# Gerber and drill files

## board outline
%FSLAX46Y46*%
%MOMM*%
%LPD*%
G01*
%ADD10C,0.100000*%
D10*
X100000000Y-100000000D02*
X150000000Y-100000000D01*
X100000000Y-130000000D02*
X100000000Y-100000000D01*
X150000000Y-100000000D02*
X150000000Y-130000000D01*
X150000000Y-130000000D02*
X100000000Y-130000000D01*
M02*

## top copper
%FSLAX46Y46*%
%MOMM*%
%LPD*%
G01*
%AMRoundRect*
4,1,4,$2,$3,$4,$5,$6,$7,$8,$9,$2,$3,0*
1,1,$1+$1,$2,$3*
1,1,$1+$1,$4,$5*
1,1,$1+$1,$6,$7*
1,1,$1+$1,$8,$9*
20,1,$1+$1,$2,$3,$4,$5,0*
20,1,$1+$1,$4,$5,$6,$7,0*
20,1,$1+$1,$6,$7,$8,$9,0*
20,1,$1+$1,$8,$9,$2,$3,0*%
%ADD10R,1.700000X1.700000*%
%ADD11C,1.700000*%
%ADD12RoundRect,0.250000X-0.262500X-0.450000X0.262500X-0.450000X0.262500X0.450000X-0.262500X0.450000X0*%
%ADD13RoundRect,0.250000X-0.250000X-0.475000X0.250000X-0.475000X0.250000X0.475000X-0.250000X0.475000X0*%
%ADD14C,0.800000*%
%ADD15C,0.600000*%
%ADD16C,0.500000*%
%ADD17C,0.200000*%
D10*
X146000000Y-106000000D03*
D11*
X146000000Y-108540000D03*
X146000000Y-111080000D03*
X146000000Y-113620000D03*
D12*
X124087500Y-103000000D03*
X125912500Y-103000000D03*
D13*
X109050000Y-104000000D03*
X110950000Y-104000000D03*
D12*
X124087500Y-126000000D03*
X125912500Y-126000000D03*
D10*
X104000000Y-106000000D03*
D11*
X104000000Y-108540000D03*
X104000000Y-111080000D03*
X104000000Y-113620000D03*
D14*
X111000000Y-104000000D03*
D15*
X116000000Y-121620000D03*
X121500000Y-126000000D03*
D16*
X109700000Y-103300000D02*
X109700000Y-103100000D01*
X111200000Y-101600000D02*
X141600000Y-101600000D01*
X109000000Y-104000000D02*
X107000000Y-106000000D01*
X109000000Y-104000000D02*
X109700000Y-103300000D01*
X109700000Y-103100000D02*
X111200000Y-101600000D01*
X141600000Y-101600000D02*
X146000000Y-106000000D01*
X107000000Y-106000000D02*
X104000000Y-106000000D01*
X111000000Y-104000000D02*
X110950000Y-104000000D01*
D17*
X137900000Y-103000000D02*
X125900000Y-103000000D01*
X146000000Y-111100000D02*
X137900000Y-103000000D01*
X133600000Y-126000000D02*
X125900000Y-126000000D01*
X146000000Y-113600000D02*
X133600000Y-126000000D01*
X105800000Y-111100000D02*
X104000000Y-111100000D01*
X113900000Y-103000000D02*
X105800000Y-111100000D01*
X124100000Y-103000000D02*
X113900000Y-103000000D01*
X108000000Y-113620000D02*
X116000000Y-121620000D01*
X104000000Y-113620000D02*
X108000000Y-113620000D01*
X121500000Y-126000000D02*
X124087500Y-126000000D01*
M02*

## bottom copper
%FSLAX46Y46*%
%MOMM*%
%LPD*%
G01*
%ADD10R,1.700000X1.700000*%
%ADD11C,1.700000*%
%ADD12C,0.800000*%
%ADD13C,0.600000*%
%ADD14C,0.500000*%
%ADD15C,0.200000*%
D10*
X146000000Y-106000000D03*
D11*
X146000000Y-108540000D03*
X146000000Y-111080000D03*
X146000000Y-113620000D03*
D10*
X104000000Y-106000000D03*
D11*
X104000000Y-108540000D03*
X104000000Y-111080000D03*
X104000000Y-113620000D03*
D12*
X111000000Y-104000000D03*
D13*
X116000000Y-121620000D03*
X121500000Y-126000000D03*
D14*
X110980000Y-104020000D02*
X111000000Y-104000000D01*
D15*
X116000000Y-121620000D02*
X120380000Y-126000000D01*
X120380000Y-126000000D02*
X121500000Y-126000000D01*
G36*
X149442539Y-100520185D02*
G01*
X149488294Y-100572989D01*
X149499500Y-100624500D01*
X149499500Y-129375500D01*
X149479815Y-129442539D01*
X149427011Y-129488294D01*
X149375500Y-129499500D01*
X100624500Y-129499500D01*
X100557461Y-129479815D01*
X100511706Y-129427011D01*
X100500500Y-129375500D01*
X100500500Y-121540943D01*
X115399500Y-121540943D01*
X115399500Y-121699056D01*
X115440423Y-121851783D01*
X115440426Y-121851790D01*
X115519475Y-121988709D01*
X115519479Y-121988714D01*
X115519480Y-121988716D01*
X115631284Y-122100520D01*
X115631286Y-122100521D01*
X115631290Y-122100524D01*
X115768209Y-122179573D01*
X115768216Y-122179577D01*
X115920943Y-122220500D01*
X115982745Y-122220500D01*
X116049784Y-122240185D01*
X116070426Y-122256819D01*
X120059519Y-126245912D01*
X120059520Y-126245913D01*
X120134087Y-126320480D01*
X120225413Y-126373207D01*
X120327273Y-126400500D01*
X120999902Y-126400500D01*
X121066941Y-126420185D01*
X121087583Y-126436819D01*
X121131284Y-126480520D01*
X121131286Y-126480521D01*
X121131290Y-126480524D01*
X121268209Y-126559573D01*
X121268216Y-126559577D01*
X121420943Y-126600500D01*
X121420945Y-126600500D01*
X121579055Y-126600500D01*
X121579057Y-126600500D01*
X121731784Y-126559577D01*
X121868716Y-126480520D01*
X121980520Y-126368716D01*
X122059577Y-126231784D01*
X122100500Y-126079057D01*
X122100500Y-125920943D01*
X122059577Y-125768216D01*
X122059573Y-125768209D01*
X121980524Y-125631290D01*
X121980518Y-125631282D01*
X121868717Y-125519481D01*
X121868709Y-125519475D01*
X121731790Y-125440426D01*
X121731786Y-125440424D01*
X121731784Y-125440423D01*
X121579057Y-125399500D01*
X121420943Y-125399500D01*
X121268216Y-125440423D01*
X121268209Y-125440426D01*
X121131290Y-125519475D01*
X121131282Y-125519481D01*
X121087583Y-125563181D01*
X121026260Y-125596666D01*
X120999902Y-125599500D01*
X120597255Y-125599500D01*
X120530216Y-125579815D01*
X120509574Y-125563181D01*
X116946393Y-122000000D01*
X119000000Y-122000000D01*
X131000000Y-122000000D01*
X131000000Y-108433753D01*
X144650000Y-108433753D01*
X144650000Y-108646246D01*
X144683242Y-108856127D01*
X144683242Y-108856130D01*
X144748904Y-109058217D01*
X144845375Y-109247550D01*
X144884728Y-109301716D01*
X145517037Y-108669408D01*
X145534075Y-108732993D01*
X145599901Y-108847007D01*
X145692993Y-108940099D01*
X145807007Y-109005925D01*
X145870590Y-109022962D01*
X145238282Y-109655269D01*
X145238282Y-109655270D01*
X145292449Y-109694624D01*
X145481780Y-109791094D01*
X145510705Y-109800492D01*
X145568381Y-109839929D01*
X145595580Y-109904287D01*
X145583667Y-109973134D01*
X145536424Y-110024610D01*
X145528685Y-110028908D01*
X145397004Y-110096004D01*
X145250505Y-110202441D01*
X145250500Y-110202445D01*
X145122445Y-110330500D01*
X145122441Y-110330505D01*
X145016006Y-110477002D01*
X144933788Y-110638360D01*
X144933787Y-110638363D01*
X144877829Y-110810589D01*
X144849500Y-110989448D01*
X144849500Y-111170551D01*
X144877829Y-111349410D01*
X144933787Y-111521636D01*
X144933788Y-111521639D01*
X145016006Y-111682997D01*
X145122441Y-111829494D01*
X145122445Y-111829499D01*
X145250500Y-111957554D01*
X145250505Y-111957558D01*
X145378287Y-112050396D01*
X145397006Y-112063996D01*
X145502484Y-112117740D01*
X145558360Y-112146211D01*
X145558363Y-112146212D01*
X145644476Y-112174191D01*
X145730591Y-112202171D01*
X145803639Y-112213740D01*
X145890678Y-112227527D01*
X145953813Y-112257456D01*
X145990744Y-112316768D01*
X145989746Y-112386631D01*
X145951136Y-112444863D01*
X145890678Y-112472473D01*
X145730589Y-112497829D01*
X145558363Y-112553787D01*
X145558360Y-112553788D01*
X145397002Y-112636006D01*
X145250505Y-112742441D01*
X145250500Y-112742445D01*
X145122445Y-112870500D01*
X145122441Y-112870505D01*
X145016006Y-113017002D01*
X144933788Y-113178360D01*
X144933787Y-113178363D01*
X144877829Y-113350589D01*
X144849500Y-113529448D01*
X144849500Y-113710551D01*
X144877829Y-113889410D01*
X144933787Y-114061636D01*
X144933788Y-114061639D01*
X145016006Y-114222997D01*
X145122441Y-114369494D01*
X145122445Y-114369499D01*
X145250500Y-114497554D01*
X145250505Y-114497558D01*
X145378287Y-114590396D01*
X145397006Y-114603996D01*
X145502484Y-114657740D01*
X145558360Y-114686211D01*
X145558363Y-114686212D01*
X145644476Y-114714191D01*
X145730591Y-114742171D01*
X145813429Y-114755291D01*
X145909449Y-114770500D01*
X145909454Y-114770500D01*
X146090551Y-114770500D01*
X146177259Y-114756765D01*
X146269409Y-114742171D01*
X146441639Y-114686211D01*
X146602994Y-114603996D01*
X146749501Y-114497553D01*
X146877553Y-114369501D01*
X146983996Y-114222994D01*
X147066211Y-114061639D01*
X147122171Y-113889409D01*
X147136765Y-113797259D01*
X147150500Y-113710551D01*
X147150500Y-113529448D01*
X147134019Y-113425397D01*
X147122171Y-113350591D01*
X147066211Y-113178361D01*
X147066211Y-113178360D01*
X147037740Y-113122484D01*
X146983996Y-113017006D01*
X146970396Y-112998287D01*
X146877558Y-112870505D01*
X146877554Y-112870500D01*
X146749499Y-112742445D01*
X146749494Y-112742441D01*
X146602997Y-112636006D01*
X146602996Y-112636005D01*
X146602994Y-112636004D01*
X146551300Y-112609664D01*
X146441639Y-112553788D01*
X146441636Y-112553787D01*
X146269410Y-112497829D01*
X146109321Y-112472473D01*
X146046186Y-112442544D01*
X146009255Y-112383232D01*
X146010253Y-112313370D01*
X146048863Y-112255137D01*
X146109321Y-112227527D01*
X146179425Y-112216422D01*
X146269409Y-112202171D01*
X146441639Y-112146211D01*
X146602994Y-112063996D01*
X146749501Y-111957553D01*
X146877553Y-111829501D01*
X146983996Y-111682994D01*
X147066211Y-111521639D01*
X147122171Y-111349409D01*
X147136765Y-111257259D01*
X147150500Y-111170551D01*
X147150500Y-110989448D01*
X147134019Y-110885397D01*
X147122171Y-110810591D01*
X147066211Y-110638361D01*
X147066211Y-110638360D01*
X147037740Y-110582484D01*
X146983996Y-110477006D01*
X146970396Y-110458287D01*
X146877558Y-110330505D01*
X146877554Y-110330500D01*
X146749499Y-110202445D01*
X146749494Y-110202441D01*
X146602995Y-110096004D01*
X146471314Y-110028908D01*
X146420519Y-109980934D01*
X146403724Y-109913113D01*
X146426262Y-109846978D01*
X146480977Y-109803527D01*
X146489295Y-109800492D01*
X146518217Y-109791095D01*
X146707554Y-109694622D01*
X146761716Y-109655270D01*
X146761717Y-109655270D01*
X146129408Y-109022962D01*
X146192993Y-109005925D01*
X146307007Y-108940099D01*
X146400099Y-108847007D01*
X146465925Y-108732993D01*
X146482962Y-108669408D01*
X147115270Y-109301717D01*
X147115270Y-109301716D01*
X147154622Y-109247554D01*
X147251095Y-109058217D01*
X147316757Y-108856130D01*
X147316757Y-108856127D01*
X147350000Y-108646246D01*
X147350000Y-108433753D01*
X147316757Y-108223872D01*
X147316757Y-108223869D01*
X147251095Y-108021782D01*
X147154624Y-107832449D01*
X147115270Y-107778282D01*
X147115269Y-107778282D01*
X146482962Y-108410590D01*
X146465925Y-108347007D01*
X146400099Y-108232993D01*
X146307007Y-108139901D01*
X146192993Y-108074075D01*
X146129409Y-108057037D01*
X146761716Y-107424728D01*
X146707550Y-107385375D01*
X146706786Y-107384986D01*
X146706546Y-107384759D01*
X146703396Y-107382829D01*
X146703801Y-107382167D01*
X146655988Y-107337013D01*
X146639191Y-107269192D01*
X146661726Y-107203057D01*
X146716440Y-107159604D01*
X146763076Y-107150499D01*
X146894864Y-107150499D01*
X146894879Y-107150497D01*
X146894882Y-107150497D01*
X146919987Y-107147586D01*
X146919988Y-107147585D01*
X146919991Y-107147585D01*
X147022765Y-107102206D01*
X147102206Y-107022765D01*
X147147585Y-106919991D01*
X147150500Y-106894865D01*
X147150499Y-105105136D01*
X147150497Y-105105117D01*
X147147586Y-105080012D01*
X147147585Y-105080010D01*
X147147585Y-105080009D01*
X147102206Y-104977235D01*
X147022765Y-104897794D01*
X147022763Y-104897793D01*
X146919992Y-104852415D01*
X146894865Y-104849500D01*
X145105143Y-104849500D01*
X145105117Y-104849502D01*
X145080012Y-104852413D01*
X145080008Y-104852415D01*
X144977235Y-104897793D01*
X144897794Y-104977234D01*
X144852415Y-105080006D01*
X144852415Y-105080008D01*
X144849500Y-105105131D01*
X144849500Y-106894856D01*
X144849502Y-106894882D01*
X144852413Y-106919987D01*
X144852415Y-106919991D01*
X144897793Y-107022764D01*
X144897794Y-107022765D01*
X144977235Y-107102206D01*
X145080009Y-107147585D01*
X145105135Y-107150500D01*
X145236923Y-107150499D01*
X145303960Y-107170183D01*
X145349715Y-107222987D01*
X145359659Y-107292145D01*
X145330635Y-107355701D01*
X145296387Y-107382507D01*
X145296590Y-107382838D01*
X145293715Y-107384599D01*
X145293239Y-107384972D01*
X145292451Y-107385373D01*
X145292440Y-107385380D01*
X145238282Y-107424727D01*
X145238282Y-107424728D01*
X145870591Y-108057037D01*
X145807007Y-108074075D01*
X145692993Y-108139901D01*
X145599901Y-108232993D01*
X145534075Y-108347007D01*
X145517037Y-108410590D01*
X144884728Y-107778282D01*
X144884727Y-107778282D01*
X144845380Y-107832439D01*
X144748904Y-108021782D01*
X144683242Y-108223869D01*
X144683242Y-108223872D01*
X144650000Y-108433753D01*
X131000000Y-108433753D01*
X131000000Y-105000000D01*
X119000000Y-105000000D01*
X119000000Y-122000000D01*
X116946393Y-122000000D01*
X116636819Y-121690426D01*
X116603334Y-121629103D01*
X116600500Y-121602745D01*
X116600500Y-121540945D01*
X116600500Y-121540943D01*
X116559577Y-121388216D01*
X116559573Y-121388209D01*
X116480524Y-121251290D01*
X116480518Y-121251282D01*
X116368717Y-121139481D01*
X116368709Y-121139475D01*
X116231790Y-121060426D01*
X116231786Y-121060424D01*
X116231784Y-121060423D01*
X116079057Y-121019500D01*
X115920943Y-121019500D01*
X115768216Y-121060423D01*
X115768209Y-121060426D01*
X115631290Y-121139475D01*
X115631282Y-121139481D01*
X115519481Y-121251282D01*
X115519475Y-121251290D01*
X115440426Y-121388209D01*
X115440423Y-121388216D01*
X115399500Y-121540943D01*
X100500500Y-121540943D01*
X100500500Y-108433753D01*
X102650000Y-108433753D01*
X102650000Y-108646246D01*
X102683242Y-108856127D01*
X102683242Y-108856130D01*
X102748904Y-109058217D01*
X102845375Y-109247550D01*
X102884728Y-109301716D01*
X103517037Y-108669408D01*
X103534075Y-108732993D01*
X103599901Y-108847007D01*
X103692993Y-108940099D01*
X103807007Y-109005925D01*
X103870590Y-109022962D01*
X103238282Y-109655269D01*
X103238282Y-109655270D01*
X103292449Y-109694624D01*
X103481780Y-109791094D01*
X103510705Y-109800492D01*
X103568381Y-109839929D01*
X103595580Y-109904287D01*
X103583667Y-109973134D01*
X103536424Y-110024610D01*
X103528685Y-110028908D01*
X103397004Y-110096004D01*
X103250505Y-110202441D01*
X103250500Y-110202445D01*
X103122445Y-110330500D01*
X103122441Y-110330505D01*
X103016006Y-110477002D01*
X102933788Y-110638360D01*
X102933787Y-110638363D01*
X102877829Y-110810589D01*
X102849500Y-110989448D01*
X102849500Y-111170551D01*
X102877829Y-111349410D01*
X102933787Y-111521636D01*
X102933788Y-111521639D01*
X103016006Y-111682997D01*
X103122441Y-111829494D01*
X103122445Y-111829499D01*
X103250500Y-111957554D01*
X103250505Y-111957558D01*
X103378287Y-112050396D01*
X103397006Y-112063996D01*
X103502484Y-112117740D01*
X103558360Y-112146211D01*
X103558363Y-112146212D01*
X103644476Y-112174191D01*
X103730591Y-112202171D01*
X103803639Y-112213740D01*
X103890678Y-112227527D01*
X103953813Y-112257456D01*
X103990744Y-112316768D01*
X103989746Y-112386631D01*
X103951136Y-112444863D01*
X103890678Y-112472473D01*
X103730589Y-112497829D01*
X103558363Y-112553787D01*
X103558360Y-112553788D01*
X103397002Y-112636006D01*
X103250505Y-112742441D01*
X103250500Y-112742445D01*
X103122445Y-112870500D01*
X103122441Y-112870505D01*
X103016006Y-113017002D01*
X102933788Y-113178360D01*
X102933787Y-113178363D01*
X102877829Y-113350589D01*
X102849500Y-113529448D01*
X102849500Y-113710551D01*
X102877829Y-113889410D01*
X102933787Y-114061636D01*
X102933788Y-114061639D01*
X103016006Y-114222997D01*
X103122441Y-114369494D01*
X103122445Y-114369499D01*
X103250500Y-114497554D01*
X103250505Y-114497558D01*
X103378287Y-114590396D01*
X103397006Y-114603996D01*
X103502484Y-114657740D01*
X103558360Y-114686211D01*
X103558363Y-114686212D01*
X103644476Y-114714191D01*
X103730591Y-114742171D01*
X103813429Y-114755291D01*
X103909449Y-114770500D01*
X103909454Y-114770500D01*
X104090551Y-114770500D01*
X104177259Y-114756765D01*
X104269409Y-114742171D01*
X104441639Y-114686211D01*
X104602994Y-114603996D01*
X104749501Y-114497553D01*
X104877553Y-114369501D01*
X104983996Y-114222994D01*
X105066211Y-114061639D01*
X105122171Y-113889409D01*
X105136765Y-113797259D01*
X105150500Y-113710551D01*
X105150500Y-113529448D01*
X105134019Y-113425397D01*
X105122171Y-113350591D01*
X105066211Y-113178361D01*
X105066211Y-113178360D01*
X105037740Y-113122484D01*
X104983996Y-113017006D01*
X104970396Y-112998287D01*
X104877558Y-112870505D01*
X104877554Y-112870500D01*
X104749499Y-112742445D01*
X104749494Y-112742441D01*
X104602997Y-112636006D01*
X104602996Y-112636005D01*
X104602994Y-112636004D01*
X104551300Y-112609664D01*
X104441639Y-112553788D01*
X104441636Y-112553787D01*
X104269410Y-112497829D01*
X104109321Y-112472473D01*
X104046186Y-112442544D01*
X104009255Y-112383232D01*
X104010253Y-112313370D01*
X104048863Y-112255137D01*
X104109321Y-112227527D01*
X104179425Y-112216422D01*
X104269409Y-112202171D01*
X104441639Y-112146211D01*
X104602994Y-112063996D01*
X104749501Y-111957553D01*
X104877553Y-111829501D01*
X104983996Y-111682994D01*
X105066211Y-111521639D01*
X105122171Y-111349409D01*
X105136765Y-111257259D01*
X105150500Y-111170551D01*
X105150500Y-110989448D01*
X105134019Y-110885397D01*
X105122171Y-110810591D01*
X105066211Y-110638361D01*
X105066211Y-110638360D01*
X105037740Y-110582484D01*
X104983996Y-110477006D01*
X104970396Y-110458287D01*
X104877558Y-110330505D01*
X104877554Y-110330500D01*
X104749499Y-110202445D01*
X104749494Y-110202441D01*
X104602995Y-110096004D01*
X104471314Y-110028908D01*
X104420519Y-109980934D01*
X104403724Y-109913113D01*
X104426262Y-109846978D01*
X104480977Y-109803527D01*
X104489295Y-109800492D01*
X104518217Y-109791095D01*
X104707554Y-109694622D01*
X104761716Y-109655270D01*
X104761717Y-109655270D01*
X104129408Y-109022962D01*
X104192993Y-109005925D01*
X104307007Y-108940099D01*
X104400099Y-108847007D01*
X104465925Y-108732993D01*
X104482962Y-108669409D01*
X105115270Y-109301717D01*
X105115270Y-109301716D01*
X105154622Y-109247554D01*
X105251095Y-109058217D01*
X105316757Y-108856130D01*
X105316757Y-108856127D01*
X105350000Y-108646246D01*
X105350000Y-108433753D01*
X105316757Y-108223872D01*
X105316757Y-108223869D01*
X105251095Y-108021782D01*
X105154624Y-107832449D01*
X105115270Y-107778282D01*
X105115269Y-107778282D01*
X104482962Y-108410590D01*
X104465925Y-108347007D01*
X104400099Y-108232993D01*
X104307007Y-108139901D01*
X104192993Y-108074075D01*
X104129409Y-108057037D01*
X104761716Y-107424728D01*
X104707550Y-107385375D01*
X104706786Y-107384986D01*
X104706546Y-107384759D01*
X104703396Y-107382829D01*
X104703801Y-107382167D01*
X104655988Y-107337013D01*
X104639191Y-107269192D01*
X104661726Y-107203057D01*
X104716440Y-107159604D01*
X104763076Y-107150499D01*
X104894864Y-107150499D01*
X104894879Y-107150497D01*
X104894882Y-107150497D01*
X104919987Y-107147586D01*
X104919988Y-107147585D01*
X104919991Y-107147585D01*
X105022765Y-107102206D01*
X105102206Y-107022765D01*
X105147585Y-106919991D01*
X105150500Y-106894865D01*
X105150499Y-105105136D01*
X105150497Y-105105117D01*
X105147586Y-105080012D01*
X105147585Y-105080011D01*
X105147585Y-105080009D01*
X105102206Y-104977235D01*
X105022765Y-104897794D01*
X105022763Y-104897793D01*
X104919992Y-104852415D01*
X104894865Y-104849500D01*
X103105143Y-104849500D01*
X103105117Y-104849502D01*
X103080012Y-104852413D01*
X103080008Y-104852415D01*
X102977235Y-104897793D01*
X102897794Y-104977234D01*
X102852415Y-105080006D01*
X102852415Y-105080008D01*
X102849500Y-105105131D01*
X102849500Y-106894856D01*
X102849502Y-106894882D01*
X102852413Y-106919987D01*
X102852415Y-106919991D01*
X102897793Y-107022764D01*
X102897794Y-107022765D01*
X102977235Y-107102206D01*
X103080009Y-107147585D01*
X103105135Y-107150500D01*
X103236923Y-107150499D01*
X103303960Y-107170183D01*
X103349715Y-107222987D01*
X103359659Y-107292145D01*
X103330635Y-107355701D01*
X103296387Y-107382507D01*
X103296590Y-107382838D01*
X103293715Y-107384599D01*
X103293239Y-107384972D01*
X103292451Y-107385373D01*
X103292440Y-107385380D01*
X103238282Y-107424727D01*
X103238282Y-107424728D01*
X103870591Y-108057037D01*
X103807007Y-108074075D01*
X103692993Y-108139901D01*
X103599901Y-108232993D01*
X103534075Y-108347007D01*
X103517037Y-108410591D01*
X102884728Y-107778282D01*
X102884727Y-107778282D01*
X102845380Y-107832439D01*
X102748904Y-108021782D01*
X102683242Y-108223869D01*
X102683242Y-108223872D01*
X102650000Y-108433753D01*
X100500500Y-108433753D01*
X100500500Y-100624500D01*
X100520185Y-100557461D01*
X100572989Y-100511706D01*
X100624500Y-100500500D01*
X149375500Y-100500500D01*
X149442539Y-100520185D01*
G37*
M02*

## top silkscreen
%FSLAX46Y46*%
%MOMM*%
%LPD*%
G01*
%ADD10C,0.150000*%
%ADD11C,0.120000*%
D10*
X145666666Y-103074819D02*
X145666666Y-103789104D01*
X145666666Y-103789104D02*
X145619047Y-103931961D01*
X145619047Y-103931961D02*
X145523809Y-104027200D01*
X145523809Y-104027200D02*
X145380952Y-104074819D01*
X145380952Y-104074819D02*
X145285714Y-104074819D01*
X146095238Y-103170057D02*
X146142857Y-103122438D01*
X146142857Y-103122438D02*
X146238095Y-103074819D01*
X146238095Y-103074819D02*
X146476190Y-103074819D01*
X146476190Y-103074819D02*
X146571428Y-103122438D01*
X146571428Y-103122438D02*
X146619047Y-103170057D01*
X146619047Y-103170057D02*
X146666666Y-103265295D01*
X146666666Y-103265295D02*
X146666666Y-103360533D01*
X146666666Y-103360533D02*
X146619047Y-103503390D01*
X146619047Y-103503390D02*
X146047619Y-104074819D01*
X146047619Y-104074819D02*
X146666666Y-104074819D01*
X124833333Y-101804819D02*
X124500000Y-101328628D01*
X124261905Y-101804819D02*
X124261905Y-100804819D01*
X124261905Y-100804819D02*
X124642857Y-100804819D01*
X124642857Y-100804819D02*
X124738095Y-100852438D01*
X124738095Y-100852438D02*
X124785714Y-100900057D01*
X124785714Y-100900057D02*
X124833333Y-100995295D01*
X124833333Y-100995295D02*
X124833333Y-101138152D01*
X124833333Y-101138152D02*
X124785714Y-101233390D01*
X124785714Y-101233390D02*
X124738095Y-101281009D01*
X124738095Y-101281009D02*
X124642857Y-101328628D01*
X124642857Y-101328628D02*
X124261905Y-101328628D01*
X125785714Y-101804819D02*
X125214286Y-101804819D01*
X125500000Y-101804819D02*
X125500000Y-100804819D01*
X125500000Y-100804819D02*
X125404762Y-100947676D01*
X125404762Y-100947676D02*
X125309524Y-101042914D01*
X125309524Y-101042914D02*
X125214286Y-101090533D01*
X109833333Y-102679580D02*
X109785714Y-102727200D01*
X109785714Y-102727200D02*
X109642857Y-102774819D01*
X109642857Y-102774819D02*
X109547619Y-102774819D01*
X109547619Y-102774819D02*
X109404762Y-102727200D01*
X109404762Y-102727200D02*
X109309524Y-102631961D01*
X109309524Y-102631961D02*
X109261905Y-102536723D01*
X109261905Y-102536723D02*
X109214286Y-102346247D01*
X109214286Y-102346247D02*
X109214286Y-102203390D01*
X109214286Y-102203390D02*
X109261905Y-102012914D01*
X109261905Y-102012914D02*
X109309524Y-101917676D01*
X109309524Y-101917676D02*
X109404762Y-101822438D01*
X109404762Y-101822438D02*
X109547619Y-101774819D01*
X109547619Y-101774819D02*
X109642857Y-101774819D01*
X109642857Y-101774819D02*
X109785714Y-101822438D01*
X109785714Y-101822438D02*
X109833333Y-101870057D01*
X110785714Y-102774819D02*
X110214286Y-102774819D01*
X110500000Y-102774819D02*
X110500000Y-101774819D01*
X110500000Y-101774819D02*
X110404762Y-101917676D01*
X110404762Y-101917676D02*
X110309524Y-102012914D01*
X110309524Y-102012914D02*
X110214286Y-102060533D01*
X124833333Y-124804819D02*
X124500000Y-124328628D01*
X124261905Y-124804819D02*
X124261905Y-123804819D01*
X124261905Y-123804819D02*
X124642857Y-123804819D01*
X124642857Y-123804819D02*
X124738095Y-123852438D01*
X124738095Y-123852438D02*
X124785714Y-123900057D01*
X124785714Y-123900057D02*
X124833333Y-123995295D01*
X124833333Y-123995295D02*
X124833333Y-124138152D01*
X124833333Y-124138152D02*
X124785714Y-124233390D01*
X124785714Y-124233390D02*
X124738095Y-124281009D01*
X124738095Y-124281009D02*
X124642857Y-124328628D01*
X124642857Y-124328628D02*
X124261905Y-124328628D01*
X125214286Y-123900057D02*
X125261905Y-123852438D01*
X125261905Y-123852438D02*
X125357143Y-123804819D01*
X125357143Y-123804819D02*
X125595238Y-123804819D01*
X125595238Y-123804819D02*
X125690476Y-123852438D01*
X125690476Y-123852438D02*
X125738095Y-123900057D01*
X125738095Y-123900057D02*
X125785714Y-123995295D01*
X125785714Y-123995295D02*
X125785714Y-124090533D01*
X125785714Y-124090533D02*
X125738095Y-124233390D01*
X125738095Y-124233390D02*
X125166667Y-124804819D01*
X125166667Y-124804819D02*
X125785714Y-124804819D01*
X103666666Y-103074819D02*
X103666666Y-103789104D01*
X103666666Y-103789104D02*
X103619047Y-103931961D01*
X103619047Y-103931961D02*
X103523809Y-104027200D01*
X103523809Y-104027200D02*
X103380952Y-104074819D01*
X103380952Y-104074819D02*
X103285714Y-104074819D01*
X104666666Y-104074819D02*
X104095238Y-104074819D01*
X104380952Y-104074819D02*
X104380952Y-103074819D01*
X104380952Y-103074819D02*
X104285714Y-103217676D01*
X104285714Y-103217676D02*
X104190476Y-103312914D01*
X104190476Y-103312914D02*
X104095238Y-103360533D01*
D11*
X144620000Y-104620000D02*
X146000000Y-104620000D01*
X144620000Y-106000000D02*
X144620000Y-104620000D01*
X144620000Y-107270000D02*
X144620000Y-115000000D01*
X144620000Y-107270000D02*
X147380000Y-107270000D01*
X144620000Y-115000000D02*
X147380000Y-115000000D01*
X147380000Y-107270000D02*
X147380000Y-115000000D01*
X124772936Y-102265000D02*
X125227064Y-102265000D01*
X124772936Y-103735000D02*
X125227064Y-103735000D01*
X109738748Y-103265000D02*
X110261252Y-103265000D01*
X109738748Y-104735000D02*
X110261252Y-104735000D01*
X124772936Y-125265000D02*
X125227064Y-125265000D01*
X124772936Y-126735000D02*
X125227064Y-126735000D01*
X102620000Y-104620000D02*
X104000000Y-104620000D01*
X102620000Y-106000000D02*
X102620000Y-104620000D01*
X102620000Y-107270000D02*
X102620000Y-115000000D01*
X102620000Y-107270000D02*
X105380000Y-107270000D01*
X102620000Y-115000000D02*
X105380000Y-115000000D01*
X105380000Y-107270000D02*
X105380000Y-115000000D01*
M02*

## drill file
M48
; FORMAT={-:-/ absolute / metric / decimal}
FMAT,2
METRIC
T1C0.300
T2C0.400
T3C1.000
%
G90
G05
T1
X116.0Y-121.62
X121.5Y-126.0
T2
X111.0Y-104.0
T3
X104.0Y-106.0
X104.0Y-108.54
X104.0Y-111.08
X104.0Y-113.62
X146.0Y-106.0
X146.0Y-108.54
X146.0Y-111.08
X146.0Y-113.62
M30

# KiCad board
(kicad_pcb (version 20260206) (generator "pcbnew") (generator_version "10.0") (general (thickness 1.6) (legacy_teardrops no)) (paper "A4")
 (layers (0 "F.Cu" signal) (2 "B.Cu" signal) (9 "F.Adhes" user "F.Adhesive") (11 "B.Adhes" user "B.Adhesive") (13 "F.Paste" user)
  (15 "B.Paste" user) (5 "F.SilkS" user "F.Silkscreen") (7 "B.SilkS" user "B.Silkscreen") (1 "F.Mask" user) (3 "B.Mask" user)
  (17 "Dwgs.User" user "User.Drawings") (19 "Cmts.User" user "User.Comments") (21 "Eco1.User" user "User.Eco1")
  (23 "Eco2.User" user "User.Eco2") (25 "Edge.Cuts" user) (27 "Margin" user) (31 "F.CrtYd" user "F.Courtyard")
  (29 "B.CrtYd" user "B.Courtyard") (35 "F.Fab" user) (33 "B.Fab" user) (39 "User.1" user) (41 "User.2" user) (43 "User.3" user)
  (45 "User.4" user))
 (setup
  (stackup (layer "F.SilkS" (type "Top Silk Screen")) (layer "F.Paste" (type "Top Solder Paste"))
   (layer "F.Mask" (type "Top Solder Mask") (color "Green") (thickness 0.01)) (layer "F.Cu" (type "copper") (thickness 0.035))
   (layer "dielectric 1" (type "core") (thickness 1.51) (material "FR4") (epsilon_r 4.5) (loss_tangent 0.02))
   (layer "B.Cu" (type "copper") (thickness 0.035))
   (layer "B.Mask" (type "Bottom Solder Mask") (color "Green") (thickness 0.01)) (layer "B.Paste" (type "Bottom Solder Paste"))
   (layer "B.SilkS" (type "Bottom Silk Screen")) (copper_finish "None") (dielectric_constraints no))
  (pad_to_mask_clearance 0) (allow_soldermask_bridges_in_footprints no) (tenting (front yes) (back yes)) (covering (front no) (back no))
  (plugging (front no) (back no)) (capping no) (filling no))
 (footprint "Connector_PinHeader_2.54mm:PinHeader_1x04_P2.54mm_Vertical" (layer "F.Cu") (at 146 106)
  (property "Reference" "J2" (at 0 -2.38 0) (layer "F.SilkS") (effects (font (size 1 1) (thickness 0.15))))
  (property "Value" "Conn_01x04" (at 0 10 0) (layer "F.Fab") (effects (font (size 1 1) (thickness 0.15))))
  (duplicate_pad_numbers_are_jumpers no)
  (fp_line (start -1.38 -1.38) (end 0 -1.38) (stroke (width 0.12) (type solid)) (layer "F.SilkS"))
  (fp_line (start -1.38 0) (end -1.38 -1.38) (stroke (width 0.12) (type solid)) (layer "F.SilkS"))
  (fp_line (start -1.38 1.27) (end -1.38 9) (stroke (width 0.12) (type solid)) (layer "F.SilkS"))
  (fp_line (start -1.38 1.27) (end 1.38 1.27) (stroke (width 0.12) (type solid)) (layer "F.SilkS"))
  (fp_line (start -1.38 9) (end 1.38 9) (stroke (width 0.12) (type solid)) (layer "F.SilkS"))
  (fp_line (start 1.38 1.27) (end 1.38 9) (stroke (width 0.12) (type solid)) (layer "F.SilkS"))
  (pad "1" thru_hole rect (at 0 0) (size 1.7 1.7) (drill 1) (layers "*.Cu" "*.Mask") (remove_unused_layers no) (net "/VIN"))
  (pad "2" thru_hole circle (at 0 2.54) (size 1.7 1.7) (drill 1) (layers "*.Cu" "*.Mask") (remove_unused_layers no) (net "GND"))
  (pad "3" thru_hole circle (at 0 5.08) (size 1.7 1.7) (drill 1) (layers "*.Cu" "*.Mask") (remove_unused_layers no) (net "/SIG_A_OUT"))
  (pad "4" thru_hole circle (at 0 7.62) (size 1.7 1.7) (drill 1) (layers "*.Cu" "*.Mask") (remove_unused_layers no) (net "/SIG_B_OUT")))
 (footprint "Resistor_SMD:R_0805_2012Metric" (layer "F.Cu") (at 125 103)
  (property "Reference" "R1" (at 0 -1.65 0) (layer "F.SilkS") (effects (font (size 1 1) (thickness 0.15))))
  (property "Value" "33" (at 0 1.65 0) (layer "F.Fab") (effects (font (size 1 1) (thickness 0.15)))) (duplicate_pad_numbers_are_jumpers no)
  (fp_line (start -0.227064 -0.735) (end 0.227064 -0.735) (stroke (width 0.12) (type solid)) (layer "F.SilkS"))
  (fp_line (start -0.227064 0.735) (end 0.227064 0.735) (stroke (width 0.12) (type solid)) (layer "F.SilkS"))
  (pad "1" smd roundrect (at -0.9125 0) (size 1.025 1.4) (layers "F.Cu" "F.Mask" "F.Paste") (roundrect_rratio 0.243902) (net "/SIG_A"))
  (pad "2" smd roundrect (at 0.9125 0) (size 1.025 1.4) (layers "F.Cu" "F.Mask" "F.Paste") (roundrect_rratio 0.243902) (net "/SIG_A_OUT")))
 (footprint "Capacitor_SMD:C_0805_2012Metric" (layer "F.Cu") (at 110 104)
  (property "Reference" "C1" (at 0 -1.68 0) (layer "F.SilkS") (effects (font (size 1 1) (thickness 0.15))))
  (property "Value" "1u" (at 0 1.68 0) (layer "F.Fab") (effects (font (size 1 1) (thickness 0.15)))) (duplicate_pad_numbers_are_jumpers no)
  (fp_line (start -0.261252 -0.735) (end 0.261252 -0.735) (stroke (width 0.12) (type solid)) (layer "F.SilkS"))
  (fp_line (start -0.261252 0.735) (end 0.261252 0.735) (stroke (width 0.12) (type solid)) (layer "F.SilkS"))
  (pad "1" smd roundrect (at -0.95 0) (size 1 1.45) (layers "F.Cu" "F.Mask" "F.Paste") (roundrect_rratio 0.25) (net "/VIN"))
  (pad "2" smd roundrect (at 0.95 0) (size 1 1.45) (layers "F.Cu" "F.Mask" "F.Paste") (roundrect_rratio 0.25) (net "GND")))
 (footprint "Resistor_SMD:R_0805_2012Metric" (layer "F.Cu") (at 125 126)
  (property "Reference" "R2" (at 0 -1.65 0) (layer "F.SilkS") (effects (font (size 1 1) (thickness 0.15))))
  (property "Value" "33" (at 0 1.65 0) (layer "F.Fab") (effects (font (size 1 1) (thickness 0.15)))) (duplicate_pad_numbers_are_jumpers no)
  (fp_line (start -0.227064 -0.735) (end 0.227064 -0.735) (stroke (width 0.12) (type solid)) (layer "F.SilkS"))
  (fp_line (start -0.227064 0.735) (end 0.227064 0.735) (stroke (width 0.12) (type solid)) (layer "F.SilkS"))
  (pad "1" smd roundrect (at -0.9125 0) (size 1.025 1.4) (layers "F.Cu" "F.Mask" "F.Paste") (roundrect_rratio 0.243902) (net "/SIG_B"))
  (pad "2" smd roundrect (at 0.9125 0) (size 1.025 1.4) (layers "F.Cu" "F.Mask" "F.Paste") (roundrect_rratio 0.243902) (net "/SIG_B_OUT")))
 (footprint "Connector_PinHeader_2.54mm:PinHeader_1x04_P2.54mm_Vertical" (layer "F.Cu") (at 104 106)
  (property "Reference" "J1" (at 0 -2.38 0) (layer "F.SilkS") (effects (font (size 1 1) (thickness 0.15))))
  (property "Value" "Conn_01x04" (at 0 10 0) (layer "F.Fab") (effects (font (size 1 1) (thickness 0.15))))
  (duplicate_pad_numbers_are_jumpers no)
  (fp_line (start -1.38 -1.38) (end 0 -1.38) (stroke (width 0.12) (type solid)) (layer "F.SilkS"))
  (fp_line (start -1.38 0) (end -1.38 -1.38) (stroke (width 0.12) (type solid)) (layer "F.SilkS"))
  (fp_line (start -1.38 1.27) (end -1.38 9) (stroke (width 0.12) (type solid)) (layer "F.SilkS"))
  (fp_line (start -1.38 1.27) (end 1.38 1.27) (stroke (width 0.12) (type solid)) (layer "F.SilkS"))
  (fp_line (start -1.38 9) (end 1.38 9) (stroke (width 0.12) (type solid)) (layer "F.SilkS"))
  (fp_line (start 1.38 1.27) (end 1.38 9) (stroke (width 0.12) (type solid)) (layer "F.SilkS"))
  (pad "1" thru_hole rect (at 0 0) (size 1.7 1.7) (drill 1) (layers "*.Cu" "*.Mask") (remove_unused_layers no) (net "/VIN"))
  (pad "2" thru_hole circle (at 0 2.54) (size 1.7 1.7) (drill 1) (layers "*.Cu" "*.Mask") (remove_unused_layers no) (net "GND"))
  (pad "3" thru_hole circle (at 0 5.08) (size 1.7 1.7) (drill 1) (layers "*.Cu" "*.Mask") (remove_unused_layers no) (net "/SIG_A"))
  (pad "4" thru_hole circle (at 0 7.62) (size 1.7 1.7) (drill 1) (layers "*.Cu" "*.Mask") (remove_unused_layers no) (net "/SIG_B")))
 (gr_line (start 100 100) (end 150 100) (stroke (width 0.1) (type default)) (layer "Edge.Cuts"))
 (gr_line (start 100 130) (end 100 100) (stroke (width 0.1) (type default)) (layer "Edge.Cuts"))
 (gr_line (start 150 100) (end 150 130) (stroke (width 0.1) (type default)) (layer "Edge.Cuts"))
 (gr_line (start 150 130) (end 100 130) (stroke (width 0.1) (type default)) (layer "Edge.Cuts"))
 (segment (start 109.7 103.3) (end 109.7 103.1) (width 0.5) (layer "F.Cu") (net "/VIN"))
 (segment (start 111.2 101.6) (end 141.6 101.6) (width 0.5) (layer "F.Cu") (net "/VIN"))
 (segment (start 109 104) (end 107 106) (width 0.5) (layer "F.Cu") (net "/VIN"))
 (segment (start 109 104) (end 109.7 103.3) (width 0.5) (layer "F.Cu") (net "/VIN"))
 (segment (start 109.7 103.1) (end 111.2 101.6) (width 0.5) (layer "F.Cu") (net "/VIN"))
 (segment (start 141.6 101.6) (end 146 106) (width 0.5) (layer "F.Cu") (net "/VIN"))
 (segment (start 107 106) (end 104 106) (width 0.5) (layer "F.Cu") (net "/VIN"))
 (segment (start 111 104) (end 110.95 104) (width 0.5) (layer "F.Cu") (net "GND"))
 (via (at 111 104) (size 0.8) (drill 0.4) (layers "F.Cu" "B.Cu") (capping yes) (filling yes) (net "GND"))
 (segment (start 110.98 104.02) (end 111 104) (width 0.5) (layer "B.Cu") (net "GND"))
 (segment (start 137.9 103) (end 125.9 103) (width 0.2) (layer "F.Cu") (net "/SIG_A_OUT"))
 (segment (start 146 111.1) (end 137.9 103) (width 0.2) (layer "F.Cu") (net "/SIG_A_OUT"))
 (segment (start 133.6 126) (end 125.9 126) (width 0.2) (layer "F.Cu") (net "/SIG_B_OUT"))
 (segment (start 146 113.6) (end 133.6 126) (width 0.2) (layer "F.Cu") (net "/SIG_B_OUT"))
 (segment (start 105.8 111.1) (end 104 111.1) (width 0.2) (layer "F.Cu") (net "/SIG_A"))
 (segment (start 113.9 103) (end 105.8 111.1) (width 0.2) (layer "F.Cu") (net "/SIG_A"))
 (segment (start 124.1 103) (end 113.9 103) (width 0.2) (layer "F.Cu") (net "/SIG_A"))
 (segment (start 108 113.62) (end 116 121.62) (width 0.2) (locked yes) (layer "F.Cu") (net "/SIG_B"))
 (segment (start 104 113.62) (end 108 113.62) (width 0.2) (locked yes) (layer "F.Cu") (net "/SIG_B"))
 (segment (start 121.5 126) (end 124.0875 126) (width 0.2) (locked yes) (layer "F.Cu") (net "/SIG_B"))
 (via (at 116 121.62) (size 0.6) (drill 0.3) (layers "F.Cu" "B.Cu") (locked yes) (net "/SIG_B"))
 (via (at 121.5 126) (size 0.6) (drill 0.3) (layers "F.Cu" "B.Cu") (locked yes) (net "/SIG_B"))
 (segment (start 116 121.62) (end 120.38 126) (width 0.2) (locked yes) (layer "B.Cu") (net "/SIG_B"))
 (segment (start 120.38 126) (end 121.5 126) (width 0.2) (locked yes) (layer "B.Cu") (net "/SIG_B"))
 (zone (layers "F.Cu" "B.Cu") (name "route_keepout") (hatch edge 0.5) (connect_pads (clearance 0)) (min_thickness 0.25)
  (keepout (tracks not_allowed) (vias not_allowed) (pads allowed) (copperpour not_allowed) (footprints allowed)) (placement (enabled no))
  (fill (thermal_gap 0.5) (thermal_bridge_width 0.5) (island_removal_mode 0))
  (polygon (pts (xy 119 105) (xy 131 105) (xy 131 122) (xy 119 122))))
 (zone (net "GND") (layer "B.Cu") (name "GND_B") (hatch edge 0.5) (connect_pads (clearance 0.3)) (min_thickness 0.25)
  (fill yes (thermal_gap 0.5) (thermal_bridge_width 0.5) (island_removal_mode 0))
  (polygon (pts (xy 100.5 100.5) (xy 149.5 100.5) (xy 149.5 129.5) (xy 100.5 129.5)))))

